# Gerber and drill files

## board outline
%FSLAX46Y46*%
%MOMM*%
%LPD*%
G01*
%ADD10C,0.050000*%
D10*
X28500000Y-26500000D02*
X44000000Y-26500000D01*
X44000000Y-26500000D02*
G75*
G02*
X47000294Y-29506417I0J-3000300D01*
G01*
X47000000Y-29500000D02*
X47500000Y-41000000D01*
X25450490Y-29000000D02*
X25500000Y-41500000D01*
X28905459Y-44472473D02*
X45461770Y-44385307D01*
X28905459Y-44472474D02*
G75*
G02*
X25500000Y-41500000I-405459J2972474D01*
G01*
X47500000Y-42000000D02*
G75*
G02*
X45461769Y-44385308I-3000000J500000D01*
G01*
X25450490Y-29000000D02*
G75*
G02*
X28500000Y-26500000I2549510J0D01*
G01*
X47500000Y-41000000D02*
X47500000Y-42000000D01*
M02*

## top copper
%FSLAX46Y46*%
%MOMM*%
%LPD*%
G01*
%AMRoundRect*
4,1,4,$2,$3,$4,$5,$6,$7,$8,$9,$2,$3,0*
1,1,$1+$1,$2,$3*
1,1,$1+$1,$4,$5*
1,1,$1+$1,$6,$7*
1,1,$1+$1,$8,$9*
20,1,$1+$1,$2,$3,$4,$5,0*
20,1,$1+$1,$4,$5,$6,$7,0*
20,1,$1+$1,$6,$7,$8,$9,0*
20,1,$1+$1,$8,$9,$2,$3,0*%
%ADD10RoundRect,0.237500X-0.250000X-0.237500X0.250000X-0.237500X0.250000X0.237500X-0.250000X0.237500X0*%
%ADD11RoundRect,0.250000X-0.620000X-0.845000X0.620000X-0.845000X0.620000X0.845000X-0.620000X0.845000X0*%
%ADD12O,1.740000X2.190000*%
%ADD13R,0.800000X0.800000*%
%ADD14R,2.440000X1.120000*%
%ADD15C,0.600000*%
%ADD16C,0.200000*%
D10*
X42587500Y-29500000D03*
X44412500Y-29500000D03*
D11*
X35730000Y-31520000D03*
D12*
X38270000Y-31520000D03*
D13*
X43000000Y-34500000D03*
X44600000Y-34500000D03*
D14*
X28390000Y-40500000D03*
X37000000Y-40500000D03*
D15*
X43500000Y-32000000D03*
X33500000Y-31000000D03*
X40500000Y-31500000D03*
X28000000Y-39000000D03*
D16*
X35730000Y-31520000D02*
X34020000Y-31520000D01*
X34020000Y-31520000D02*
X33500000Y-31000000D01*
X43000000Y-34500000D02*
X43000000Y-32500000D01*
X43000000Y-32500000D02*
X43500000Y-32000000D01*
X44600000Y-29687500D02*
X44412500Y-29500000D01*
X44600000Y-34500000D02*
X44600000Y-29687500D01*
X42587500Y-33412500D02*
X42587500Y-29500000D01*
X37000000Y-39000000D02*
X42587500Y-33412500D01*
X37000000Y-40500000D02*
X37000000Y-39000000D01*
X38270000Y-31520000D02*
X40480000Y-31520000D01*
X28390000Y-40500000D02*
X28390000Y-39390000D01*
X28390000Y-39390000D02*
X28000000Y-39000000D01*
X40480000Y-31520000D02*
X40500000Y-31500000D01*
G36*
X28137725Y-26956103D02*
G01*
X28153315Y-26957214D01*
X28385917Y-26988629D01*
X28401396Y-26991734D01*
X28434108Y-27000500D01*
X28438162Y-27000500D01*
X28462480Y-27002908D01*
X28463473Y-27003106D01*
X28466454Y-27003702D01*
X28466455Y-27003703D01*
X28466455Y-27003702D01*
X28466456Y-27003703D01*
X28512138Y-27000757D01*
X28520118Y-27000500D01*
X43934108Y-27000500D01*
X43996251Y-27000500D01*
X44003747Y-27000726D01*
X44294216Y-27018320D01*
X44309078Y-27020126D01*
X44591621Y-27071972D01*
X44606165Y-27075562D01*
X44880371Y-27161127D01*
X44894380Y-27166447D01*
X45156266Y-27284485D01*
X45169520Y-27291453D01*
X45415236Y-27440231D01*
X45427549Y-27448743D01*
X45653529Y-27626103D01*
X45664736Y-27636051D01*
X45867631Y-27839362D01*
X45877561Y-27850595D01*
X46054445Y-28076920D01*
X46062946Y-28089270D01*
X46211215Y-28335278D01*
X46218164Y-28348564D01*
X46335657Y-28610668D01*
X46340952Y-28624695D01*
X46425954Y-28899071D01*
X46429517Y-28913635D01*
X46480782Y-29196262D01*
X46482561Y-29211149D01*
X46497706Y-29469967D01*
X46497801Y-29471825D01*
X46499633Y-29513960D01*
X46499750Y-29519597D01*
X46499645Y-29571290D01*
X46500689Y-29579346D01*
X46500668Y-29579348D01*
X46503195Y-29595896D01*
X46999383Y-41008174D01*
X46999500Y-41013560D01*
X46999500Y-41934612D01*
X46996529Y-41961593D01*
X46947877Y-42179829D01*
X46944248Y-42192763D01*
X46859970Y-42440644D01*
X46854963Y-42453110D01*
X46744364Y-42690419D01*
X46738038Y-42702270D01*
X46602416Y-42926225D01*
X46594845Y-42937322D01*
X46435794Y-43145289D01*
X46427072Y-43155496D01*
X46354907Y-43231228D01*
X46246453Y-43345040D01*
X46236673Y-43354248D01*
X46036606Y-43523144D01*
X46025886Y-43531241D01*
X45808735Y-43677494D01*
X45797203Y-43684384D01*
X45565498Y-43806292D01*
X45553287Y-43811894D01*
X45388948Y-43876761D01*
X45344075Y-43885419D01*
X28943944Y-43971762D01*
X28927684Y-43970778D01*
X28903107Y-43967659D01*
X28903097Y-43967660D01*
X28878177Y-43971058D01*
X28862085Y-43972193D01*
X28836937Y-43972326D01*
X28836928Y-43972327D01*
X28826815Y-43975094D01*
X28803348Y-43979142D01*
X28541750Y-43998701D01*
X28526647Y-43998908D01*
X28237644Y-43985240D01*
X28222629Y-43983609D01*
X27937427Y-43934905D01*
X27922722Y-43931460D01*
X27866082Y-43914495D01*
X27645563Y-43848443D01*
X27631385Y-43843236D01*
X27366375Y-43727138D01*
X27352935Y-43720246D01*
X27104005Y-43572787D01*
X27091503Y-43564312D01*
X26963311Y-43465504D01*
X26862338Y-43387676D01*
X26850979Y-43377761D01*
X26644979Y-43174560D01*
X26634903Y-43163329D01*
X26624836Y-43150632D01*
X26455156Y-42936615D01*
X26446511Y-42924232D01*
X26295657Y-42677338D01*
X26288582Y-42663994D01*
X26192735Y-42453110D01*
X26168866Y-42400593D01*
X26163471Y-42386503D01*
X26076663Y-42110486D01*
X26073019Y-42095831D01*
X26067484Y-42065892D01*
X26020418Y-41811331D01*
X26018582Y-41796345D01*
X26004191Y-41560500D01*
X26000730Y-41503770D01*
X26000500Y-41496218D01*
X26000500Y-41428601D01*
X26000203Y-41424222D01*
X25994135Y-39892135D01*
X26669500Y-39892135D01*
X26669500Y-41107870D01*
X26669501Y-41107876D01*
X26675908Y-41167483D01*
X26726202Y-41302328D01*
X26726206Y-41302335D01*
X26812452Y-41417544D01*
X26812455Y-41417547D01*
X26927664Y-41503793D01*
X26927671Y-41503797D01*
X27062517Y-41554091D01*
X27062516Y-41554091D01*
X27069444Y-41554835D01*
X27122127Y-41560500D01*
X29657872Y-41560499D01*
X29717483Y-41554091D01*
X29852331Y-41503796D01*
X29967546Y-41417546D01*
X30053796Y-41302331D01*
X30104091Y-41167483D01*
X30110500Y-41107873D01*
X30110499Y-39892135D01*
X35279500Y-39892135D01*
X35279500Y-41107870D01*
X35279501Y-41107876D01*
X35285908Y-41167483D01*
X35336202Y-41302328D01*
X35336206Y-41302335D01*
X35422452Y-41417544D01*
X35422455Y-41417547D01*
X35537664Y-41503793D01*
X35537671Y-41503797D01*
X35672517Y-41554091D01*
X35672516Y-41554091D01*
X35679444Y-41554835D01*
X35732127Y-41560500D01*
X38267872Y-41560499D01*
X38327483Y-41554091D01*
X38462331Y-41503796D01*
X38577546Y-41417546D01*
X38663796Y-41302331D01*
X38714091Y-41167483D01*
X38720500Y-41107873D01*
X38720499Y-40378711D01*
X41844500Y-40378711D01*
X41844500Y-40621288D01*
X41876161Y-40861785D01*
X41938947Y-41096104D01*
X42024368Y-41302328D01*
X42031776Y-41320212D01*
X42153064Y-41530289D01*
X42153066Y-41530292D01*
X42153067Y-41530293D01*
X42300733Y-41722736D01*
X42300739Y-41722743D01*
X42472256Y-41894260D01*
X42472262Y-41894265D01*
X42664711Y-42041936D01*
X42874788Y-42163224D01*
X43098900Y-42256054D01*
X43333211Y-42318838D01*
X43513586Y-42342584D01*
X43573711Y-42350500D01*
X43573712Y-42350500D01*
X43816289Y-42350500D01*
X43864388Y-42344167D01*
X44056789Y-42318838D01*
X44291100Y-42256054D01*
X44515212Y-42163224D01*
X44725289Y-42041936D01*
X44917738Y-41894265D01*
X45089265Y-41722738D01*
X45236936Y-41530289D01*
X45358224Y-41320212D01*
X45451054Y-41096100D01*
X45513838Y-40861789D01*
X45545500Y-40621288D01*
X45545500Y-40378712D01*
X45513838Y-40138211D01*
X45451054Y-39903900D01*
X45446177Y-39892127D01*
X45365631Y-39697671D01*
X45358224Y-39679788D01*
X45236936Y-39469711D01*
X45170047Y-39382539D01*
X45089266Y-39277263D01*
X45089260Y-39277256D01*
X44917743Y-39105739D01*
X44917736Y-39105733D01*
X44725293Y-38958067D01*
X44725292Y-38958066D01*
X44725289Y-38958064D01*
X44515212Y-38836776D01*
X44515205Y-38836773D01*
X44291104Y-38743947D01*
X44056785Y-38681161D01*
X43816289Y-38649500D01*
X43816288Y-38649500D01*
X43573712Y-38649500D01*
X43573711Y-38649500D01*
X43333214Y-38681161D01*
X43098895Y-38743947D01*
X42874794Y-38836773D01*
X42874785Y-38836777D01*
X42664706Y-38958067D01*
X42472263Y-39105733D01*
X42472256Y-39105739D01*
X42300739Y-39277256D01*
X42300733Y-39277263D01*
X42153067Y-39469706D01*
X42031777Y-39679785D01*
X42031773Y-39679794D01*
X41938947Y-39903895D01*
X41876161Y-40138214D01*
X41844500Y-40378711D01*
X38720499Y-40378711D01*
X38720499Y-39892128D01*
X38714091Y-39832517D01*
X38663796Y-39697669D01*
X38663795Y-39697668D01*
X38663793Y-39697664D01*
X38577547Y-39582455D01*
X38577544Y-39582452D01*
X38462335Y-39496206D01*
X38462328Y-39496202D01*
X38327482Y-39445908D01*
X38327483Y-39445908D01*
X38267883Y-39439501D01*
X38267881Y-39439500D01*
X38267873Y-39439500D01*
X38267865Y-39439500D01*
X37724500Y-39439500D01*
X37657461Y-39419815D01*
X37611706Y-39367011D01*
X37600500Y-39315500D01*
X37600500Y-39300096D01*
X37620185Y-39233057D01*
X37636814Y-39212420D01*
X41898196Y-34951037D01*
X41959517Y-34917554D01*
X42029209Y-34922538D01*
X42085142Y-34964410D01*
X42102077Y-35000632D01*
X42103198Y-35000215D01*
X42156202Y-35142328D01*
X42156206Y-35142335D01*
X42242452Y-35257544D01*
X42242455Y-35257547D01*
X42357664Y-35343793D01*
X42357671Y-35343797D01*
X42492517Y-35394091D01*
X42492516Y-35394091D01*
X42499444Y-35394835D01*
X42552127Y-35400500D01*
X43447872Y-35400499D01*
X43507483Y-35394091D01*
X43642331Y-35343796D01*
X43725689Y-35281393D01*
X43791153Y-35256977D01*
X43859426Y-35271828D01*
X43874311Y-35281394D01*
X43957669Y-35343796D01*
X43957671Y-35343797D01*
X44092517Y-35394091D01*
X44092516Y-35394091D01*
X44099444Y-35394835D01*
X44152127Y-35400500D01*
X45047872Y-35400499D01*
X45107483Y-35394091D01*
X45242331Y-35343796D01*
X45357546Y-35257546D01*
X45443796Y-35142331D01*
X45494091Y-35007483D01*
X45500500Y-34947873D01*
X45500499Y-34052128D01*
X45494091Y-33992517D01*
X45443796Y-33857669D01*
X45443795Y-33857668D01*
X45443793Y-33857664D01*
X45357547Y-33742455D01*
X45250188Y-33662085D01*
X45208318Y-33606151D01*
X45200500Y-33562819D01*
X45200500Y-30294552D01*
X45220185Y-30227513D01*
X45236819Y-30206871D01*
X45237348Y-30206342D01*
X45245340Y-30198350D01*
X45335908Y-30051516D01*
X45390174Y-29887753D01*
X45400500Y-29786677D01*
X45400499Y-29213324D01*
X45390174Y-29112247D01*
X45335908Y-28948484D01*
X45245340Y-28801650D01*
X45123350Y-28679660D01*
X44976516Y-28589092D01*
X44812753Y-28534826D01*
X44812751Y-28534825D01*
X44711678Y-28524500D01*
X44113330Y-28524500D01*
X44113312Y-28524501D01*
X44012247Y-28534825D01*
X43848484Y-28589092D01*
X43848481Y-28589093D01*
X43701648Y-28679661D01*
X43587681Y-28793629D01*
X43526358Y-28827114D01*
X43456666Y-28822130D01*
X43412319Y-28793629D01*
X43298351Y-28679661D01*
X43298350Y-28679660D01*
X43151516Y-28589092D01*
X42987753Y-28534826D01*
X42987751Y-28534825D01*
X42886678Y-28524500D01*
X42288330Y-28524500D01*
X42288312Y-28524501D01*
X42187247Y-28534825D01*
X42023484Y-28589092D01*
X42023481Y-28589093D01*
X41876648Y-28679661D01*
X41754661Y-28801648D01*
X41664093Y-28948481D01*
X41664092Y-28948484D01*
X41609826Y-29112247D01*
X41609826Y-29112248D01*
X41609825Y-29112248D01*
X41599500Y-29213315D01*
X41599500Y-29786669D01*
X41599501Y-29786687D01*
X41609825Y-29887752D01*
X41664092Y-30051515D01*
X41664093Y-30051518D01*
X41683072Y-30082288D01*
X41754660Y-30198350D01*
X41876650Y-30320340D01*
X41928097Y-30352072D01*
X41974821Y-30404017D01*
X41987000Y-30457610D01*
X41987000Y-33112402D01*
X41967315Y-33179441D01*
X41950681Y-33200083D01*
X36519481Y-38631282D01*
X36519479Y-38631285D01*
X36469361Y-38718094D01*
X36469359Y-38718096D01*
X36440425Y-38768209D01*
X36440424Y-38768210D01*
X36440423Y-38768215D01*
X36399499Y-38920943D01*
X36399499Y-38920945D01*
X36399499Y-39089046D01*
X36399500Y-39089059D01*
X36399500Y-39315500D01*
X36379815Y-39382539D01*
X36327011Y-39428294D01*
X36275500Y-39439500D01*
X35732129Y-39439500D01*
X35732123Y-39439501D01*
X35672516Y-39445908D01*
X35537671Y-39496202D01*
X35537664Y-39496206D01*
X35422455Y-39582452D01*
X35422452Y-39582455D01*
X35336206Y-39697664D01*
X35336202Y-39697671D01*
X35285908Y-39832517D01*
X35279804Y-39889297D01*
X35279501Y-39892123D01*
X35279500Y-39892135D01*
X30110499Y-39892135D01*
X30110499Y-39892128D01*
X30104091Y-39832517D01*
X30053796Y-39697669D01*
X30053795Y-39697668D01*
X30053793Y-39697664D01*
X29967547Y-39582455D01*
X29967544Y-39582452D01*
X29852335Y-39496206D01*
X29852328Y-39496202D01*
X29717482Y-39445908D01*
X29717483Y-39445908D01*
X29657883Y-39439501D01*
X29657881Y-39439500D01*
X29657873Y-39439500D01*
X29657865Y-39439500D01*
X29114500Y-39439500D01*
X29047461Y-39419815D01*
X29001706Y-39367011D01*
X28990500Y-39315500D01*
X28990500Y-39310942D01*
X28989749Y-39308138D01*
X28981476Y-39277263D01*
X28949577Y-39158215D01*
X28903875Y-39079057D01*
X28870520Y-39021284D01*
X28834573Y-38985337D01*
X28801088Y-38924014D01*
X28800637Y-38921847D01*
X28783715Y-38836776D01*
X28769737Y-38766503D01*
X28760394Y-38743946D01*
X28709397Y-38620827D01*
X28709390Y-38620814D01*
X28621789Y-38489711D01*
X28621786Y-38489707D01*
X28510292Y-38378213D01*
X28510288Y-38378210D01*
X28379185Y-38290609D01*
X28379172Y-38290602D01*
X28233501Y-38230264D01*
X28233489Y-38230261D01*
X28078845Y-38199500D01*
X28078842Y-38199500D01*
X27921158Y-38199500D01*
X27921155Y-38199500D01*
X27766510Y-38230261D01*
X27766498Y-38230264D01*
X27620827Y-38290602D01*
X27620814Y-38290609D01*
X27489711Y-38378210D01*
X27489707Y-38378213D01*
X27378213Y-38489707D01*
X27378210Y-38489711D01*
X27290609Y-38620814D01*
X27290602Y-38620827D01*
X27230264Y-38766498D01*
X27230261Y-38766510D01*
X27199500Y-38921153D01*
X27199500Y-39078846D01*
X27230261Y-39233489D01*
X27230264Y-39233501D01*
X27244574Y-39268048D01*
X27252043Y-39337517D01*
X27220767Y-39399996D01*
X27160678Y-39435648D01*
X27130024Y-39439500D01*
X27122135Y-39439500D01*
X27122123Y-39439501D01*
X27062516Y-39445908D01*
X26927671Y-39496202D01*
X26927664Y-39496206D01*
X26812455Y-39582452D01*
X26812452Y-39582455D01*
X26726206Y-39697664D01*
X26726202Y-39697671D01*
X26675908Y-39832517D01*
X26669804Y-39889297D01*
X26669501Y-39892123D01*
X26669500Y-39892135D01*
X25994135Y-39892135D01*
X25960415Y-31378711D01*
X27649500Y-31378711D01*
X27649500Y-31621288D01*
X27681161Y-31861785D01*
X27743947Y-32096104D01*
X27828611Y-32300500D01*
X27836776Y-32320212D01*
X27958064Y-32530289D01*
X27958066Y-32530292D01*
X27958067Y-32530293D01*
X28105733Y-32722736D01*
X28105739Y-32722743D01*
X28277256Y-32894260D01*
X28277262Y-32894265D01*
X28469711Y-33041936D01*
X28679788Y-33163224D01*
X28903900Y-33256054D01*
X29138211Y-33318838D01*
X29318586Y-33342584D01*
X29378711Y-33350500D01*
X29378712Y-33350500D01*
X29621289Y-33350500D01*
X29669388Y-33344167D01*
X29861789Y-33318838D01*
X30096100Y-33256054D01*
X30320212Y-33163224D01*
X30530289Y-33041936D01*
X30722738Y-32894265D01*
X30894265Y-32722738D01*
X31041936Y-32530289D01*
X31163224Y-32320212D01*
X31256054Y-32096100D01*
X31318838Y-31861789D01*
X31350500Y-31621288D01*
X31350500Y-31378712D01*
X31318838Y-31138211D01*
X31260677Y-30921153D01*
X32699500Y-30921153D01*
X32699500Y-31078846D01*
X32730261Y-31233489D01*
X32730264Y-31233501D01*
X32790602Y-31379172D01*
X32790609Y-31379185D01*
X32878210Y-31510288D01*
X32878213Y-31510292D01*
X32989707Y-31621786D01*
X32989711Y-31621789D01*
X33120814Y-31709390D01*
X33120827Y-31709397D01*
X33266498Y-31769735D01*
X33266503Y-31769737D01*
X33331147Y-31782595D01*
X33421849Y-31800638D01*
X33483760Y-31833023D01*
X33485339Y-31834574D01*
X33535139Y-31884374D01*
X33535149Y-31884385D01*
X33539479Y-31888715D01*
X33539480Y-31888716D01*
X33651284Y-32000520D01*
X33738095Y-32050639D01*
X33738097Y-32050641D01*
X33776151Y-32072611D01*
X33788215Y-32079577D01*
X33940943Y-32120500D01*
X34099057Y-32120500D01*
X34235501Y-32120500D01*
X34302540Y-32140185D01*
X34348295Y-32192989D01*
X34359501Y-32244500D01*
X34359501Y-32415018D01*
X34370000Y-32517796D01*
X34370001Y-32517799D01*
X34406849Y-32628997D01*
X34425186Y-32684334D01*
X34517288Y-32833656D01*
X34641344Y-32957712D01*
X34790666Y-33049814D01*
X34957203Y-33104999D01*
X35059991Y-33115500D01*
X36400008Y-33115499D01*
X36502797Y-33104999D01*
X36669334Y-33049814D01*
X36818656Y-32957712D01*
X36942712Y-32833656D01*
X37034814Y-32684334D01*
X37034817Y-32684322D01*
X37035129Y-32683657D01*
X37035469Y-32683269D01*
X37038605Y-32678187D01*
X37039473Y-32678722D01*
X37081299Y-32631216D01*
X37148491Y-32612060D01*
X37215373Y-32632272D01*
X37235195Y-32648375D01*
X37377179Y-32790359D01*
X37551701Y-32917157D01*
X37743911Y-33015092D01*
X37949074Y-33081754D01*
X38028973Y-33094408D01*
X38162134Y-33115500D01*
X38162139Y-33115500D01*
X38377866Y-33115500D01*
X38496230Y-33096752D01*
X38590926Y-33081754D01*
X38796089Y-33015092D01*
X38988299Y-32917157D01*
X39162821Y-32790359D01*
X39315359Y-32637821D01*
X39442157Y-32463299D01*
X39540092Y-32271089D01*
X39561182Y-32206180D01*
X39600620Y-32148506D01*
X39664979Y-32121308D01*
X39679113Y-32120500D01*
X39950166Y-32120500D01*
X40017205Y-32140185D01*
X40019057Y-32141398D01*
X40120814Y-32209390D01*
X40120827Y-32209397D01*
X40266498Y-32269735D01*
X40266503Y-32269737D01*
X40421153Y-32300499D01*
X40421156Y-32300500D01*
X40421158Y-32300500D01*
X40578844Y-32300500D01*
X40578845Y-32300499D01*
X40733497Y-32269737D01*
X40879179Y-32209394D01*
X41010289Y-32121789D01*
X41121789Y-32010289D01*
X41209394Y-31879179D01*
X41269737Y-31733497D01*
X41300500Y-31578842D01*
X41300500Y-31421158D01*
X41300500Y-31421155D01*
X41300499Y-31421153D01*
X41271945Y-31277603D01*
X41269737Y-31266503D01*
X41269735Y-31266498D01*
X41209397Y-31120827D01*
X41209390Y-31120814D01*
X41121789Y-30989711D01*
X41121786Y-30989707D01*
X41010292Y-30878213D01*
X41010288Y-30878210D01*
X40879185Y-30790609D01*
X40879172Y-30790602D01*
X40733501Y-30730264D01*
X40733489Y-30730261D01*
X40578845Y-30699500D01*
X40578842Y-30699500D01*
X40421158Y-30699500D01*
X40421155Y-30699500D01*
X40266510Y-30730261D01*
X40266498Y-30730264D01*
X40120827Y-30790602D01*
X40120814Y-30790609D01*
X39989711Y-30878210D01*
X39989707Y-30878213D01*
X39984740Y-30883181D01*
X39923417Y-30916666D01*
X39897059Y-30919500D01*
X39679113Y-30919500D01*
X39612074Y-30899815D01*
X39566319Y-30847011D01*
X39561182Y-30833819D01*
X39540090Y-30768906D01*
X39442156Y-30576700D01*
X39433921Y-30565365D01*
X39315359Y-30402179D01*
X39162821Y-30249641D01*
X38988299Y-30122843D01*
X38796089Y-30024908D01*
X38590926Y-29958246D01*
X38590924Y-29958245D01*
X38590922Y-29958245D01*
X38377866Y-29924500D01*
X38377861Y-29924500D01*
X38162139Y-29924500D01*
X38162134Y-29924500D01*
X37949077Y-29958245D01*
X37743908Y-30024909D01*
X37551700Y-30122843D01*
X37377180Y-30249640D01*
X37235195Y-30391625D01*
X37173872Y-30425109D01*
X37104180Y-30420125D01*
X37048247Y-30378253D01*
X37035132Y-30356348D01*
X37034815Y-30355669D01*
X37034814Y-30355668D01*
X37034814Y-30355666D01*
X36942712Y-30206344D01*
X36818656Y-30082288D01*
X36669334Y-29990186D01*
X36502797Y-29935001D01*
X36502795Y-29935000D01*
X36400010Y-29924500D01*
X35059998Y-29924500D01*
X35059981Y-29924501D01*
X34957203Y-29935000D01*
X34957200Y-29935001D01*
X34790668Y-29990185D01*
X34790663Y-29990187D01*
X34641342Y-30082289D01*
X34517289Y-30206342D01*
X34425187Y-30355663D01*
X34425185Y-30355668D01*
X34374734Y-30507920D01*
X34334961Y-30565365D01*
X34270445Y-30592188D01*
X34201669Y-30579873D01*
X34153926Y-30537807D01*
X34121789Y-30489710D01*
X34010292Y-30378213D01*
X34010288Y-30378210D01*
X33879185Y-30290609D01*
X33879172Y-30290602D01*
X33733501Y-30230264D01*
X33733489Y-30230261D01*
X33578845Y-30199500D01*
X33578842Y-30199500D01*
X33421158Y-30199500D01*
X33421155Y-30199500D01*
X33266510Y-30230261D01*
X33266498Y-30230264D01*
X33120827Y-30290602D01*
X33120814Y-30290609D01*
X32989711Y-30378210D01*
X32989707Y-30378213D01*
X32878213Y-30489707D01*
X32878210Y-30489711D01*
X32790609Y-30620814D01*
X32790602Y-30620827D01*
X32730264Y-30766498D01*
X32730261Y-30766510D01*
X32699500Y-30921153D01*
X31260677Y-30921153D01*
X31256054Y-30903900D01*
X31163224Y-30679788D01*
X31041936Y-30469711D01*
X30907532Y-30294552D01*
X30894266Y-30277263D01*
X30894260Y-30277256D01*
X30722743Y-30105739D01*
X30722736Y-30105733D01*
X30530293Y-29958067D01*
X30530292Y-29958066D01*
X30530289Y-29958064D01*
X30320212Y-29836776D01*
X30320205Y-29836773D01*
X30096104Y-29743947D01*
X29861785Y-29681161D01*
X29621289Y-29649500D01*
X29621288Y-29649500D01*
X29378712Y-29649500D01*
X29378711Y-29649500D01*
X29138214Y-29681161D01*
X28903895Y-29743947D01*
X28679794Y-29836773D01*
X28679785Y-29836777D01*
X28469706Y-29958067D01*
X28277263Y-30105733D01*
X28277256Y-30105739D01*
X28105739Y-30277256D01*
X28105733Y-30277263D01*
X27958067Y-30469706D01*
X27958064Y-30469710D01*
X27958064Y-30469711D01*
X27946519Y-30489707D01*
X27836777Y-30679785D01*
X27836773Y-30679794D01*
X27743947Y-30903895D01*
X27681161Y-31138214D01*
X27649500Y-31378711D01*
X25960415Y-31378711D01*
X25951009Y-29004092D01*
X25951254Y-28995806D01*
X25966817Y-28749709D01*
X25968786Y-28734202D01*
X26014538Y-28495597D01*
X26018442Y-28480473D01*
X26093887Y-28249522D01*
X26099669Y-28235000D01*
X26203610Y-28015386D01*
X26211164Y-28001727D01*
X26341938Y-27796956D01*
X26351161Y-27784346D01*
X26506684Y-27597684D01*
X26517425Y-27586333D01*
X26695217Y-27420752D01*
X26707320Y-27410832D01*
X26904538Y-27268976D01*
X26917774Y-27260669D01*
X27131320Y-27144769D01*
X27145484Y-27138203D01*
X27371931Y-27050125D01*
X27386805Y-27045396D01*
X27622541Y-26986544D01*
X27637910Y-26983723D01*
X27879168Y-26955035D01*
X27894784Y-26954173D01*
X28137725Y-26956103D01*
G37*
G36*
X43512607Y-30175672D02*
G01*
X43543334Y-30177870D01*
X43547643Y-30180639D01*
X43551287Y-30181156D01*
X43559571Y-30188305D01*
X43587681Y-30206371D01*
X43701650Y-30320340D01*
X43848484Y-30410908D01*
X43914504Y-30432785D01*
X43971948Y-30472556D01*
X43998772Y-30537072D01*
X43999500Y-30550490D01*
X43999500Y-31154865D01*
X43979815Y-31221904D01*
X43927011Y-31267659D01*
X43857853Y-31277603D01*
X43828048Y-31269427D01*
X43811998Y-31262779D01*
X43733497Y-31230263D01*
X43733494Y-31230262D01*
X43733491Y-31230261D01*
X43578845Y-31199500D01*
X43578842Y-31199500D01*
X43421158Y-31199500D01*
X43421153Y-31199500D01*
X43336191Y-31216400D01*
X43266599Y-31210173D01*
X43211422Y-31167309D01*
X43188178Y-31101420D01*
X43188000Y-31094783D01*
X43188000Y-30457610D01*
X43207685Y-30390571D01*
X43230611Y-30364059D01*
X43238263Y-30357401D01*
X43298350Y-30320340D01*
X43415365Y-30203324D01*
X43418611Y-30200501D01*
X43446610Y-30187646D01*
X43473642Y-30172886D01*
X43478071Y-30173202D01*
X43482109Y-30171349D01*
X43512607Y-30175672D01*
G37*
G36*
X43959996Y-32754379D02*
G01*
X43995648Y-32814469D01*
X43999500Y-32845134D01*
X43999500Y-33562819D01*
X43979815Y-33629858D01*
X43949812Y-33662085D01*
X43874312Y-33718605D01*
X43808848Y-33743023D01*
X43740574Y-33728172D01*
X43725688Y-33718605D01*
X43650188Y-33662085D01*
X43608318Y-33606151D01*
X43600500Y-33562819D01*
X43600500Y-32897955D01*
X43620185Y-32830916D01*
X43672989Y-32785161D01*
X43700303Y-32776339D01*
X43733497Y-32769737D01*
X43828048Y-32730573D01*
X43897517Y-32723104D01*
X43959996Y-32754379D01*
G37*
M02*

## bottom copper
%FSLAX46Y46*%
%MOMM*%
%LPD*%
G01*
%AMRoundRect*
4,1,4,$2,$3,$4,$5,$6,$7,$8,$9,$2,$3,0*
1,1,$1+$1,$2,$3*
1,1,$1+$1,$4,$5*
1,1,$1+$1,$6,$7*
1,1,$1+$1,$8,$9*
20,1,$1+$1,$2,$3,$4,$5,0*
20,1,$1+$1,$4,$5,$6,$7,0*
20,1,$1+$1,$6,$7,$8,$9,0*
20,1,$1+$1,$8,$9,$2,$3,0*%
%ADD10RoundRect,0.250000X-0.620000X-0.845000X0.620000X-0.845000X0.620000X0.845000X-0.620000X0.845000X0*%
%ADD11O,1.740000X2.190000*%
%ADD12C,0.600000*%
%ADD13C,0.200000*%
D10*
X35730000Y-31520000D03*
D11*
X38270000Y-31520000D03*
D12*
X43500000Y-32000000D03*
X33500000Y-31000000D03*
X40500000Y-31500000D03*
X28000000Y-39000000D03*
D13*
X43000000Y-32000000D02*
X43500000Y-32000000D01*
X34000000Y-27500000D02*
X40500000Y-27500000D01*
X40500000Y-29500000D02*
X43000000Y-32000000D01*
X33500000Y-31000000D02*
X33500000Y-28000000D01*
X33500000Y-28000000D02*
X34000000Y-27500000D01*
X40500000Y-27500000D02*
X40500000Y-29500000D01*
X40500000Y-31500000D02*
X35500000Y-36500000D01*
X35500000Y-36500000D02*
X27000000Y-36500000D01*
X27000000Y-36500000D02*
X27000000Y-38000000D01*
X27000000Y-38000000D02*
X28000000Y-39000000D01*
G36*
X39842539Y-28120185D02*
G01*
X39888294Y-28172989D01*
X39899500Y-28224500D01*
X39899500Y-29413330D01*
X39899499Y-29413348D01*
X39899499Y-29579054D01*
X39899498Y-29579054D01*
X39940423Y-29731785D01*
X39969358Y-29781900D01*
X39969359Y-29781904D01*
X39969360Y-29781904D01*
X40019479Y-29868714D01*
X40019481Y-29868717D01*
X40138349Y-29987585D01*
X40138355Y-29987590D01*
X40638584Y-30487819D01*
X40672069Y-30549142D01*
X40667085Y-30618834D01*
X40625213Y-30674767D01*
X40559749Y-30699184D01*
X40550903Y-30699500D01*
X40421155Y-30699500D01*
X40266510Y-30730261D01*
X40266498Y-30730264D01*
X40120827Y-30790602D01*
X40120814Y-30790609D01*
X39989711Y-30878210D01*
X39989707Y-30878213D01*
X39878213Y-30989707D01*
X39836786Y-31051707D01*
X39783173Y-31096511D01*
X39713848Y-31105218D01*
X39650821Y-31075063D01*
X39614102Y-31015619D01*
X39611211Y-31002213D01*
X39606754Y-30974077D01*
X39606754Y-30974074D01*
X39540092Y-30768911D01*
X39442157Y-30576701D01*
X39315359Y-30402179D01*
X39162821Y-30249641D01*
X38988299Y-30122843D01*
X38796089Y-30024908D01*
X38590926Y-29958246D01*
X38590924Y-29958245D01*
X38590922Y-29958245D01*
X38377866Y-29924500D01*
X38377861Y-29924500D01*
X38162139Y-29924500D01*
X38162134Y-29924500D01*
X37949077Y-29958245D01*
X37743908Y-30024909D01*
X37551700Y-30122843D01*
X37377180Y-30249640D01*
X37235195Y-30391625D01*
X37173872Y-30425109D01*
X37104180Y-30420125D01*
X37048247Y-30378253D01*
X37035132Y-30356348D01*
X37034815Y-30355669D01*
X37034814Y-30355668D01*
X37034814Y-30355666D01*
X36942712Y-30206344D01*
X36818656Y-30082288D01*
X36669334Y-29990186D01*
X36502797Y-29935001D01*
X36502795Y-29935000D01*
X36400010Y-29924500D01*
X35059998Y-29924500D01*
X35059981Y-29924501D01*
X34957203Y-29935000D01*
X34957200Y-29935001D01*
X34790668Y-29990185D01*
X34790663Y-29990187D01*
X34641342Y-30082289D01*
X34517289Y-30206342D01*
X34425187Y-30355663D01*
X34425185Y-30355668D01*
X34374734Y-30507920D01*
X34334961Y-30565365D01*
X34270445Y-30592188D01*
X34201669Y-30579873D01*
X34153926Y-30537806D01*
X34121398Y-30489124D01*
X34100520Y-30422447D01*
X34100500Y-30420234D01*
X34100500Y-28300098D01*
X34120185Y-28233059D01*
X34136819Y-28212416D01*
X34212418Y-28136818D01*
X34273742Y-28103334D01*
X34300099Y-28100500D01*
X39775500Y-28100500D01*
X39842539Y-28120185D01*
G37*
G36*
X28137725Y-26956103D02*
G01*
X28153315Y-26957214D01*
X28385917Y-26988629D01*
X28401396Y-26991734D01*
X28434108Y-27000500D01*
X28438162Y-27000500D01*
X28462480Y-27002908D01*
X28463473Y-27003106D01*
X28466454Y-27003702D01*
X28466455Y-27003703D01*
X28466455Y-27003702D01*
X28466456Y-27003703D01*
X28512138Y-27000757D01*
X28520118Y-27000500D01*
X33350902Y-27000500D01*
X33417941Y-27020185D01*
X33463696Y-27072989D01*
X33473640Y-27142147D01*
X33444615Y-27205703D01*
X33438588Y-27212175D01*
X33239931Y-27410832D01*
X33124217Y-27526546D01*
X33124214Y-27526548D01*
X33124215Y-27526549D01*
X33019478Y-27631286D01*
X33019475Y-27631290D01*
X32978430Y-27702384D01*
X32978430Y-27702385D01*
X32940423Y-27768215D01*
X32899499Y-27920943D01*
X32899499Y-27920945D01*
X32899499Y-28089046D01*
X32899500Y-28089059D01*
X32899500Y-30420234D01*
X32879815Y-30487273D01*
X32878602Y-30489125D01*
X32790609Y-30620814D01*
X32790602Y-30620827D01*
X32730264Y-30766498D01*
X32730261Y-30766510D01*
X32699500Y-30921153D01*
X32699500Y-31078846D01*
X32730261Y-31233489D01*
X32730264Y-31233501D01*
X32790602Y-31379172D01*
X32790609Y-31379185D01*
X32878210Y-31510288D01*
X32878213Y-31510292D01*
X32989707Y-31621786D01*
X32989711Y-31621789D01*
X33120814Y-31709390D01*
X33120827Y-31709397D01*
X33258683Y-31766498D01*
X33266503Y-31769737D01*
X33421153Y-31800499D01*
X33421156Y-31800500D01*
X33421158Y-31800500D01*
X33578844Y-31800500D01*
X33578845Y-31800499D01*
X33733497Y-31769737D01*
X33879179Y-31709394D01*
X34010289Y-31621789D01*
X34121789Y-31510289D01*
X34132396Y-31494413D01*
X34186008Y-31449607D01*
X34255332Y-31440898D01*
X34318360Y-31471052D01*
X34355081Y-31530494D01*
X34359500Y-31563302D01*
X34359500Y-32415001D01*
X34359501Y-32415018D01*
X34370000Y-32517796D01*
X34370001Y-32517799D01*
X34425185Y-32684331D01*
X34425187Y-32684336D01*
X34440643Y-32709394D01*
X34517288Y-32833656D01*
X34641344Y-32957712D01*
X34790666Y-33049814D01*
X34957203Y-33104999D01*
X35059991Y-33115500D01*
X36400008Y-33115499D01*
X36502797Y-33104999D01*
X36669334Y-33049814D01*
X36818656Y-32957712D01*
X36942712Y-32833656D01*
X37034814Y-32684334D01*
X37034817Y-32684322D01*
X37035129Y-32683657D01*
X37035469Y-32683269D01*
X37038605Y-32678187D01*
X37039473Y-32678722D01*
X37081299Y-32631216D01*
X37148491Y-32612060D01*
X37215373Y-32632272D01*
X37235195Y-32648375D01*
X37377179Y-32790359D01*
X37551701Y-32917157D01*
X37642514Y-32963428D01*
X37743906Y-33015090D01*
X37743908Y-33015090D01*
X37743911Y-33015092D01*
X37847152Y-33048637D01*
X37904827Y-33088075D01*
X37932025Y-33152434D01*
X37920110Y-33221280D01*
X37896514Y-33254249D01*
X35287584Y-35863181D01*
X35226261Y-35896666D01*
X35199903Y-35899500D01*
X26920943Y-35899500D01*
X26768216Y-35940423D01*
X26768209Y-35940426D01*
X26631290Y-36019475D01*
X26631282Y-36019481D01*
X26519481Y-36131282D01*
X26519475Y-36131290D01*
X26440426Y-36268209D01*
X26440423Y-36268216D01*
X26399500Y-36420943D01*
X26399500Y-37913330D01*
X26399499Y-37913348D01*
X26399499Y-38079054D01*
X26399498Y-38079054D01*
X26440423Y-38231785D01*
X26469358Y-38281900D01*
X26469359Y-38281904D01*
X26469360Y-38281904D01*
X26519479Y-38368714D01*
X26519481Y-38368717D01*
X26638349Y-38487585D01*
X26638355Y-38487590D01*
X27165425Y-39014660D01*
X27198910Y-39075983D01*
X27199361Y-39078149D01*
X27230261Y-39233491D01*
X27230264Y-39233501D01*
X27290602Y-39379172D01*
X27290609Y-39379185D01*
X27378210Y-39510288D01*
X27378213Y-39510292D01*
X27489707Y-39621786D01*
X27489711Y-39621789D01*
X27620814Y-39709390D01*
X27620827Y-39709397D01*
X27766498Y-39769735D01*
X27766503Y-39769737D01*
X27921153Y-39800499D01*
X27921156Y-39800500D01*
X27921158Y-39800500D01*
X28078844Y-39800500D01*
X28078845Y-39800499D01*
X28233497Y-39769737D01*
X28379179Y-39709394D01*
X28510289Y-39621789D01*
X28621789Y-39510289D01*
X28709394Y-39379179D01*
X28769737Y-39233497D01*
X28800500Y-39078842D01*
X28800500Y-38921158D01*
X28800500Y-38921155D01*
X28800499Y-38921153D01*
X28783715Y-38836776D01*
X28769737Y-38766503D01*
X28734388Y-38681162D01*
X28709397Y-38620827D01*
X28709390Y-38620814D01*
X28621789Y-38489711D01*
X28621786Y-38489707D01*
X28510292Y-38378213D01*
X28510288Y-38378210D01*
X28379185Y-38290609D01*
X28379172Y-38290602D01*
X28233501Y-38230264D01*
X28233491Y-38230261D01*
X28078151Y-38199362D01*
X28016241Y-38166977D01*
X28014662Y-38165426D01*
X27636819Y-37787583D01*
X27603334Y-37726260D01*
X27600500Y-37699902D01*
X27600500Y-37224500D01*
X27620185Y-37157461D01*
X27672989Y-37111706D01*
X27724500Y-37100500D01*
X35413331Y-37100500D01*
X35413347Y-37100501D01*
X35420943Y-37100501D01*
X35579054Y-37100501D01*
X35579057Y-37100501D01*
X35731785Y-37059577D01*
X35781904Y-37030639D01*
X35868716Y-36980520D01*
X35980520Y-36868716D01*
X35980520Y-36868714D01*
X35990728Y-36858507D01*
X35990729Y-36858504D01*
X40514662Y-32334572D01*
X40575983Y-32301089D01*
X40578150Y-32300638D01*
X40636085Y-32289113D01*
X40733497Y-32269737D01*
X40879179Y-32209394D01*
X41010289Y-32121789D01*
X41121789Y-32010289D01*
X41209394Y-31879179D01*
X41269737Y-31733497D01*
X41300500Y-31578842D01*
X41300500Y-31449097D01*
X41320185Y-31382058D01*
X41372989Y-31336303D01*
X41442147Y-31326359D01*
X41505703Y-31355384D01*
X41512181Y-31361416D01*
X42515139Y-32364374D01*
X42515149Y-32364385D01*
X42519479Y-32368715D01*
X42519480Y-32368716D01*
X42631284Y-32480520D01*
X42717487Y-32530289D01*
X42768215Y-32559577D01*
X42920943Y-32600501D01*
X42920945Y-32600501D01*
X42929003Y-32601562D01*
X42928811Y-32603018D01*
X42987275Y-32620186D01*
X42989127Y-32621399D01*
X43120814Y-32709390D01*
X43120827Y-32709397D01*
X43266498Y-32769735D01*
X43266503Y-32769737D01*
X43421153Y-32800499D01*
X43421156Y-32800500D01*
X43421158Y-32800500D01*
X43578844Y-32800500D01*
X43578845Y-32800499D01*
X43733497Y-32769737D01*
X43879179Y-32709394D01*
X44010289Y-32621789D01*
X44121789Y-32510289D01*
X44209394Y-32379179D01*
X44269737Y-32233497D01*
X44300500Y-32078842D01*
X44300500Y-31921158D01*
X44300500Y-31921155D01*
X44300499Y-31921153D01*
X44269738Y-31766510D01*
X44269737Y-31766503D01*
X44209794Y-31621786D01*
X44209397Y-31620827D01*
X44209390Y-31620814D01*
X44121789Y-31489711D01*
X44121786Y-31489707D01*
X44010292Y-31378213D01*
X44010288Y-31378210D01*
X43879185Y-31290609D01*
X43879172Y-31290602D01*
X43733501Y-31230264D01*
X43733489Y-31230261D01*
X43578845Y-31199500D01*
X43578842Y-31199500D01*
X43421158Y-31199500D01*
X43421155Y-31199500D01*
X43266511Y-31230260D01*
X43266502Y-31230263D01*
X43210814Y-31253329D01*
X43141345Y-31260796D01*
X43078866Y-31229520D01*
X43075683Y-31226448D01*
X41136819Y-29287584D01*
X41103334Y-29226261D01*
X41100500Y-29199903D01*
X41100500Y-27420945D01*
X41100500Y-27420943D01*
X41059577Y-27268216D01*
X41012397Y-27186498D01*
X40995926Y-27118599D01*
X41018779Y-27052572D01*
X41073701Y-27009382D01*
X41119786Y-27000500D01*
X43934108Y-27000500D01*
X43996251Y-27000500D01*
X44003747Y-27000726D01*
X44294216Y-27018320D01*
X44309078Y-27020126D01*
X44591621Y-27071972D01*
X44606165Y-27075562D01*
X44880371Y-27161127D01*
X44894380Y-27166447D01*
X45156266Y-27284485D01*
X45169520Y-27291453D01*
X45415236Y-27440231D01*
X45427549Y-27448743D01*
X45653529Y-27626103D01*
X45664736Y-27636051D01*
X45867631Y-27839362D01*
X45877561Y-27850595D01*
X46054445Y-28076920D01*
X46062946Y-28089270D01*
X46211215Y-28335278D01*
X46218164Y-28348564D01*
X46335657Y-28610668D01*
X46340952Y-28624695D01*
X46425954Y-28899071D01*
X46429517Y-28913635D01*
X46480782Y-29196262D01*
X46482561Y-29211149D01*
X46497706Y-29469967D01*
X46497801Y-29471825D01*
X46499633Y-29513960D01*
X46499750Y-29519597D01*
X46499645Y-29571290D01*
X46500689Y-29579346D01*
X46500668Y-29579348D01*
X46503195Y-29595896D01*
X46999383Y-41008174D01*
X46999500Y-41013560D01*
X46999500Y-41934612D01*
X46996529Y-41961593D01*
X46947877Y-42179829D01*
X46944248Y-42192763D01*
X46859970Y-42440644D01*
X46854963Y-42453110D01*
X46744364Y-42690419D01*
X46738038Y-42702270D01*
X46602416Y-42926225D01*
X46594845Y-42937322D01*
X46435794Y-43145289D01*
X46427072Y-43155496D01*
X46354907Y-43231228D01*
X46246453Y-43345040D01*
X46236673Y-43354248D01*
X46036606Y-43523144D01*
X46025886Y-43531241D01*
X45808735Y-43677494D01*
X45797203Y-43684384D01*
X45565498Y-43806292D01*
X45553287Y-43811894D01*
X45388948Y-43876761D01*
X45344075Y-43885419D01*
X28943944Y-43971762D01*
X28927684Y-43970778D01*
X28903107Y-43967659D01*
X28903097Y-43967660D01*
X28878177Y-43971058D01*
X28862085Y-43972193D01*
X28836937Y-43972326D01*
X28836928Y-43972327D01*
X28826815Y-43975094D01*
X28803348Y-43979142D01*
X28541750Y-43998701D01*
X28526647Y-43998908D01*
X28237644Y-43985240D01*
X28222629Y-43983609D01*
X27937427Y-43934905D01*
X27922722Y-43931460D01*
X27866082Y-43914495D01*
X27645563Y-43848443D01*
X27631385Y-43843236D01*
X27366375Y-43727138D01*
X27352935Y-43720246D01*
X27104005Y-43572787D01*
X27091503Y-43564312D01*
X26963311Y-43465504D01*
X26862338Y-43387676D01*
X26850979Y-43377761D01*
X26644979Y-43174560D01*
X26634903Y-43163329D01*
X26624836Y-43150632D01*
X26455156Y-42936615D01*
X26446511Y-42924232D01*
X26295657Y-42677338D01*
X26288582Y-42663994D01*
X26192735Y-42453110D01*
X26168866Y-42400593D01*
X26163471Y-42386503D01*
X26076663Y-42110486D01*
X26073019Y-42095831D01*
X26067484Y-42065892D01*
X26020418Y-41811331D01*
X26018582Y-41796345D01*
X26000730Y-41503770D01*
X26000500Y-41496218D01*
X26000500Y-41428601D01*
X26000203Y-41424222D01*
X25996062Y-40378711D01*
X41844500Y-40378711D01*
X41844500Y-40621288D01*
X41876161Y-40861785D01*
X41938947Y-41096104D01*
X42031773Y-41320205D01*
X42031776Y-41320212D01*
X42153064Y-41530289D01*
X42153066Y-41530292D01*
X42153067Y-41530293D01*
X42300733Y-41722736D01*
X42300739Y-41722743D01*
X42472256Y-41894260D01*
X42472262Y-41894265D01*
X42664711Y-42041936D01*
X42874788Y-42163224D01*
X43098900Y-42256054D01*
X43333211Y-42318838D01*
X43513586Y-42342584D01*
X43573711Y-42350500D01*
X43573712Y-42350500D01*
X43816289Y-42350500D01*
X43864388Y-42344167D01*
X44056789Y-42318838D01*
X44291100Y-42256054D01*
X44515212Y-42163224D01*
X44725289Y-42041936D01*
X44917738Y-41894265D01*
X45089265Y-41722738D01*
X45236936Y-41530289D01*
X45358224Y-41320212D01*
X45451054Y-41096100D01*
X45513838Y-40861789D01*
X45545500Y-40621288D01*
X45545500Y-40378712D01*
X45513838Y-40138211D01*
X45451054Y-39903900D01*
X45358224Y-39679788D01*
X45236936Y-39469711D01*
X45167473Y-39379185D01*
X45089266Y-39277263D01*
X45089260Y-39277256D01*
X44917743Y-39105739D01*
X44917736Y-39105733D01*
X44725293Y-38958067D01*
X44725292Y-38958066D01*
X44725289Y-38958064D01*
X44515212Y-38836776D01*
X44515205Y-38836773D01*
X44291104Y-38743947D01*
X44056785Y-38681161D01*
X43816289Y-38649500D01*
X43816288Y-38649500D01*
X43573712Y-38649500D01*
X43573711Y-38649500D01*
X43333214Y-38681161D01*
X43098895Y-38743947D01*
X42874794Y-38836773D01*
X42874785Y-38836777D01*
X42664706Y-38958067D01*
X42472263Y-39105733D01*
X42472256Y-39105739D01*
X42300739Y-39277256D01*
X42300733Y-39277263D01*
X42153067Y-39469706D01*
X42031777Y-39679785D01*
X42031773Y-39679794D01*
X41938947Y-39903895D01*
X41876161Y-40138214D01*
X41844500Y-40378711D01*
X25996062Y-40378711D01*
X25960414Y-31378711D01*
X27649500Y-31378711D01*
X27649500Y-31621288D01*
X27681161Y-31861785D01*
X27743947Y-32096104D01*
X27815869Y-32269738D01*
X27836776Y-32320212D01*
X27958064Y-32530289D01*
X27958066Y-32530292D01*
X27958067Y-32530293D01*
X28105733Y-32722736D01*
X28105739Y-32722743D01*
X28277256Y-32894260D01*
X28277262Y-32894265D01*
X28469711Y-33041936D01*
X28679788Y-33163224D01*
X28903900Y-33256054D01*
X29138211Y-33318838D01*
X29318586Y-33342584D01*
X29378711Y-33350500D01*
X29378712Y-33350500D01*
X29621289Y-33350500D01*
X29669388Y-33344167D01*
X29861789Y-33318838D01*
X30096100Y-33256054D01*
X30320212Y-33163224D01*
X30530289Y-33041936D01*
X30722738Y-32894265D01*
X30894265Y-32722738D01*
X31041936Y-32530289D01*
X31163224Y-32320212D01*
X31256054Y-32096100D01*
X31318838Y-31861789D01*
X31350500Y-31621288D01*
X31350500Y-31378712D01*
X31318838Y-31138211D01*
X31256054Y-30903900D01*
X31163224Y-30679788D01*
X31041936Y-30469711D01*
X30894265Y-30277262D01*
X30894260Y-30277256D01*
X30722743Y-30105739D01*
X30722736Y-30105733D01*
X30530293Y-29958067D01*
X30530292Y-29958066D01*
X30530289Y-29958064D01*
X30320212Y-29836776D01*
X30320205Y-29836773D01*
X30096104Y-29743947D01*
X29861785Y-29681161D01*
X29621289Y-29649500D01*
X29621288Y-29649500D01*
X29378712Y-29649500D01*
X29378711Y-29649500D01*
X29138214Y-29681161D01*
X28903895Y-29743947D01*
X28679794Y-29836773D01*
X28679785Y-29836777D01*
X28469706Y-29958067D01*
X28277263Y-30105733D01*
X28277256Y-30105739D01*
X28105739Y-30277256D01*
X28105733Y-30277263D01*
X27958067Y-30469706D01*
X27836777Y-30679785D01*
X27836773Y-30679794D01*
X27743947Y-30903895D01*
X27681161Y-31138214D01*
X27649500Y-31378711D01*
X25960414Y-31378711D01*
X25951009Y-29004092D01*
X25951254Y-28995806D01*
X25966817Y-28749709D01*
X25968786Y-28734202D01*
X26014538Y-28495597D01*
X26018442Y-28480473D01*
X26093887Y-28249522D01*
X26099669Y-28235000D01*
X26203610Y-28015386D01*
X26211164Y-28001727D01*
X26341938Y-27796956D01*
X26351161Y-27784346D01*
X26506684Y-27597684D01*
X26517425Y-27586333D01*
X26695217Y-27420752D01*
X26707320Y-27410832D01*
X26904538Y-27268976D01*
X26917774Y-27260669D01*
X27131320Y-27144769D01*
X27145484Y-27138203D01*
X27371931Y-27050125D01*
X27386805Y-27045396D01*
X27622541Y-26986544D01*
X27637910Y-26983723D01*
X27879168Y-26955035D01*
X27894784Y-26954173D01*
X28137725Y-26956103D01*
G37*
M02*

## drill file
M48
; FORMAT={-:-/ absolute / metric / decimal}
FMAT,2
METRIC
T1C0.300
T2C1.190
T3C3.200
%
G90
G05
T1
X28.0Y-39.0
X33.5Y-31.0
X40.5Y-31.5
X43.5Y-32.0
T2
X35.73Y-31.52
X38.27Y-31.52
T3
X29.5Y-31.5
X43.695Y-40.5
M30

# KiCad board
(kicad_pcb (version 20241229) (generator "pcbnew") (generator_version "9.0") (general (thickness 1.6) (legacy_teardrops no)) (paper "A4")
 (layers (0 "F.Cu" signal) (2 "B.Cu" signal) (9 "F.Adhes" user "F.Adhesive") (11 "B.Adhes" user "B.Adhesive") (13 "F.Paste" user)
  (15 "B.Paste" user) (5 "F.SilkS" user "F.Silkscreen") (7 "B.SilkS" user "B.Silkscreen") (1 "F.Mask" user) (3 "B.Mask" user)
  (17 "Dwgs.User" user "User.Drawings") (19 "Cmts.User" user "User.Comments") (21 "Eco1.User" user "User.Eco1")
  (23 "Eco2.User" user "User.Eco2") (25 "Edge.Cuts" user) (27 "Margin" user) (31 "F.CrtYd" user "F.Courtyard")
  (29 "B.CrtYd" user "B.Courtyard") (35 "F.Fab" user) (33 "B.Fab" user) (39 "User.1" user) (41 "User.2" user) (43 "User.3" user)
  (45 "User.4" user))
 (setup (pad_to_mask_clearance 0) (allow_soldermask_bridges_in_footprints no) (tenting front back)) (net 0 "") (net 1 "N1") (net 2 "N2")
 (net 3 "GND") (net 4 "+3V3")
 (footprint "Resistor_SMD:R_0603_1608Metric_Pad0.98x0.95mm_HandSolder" (layer "F.Cu") (at 43.5 29.5)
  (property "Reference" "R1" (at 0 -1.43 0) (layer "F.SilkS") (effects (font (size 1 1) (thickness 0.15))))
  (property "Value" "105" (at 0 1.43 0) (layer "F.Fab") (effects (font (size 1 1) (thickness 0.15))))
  (pad "1" smd roundrect (at -0.9125 0) (size 0.975 0.95) (layers "F.Cu" "F.Mask" "F.Paste") (roundrect_rratio 0.25) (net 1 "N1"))
  (pad "2" smd roundrect (at 0.9125 0) (size 0.975 0.95) (layers "F.Cu" "F.Mask" "F.Paste") (roundrect_rratio 0.25) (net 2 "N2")))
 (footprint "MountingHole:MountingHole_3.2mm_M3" (layer "F.Cu") (at 43.695 40.5)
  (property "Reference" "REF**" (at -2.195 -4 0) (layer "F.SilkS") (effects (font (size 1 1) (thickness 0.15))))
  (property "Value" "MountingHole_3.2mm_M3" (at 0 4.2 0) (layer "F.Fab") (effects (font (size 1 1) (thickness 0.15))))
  (pad "" np_thru_hole circle (at 0 0) (size 3.2 3.2) (drill 3.2) (layers "*.Cu" "*.Mask")))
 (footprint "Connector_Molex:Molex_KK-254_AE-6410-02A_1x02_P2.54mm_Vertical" (layer "F.Cu") (at 35.73 31.52)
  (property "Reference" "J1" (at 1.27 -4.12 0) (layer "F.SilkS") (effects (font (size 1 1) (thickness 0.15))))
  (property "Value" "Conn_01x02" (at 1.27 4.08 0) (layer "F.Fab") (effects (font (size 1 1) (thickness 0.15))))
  (pad "1" thru_hole roundrect (at 0 0) (size 1.74 2.19) (drill 1.19) (layers "*.Cu" "*.Mask") (remove_unused_layers no)
   (roundrect_rratio 0.143678) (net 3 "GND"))
  (pad "2" thru_hole oval (at 2.54 0) (size 1.74 2.19) (drill 1.19) (layers "*.Cu" "*.Mask") (remove_unused_layers no) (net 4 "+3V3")))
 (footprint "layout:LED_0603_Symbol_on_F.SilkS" (layer "F.Cu") (at 43.8 34.5)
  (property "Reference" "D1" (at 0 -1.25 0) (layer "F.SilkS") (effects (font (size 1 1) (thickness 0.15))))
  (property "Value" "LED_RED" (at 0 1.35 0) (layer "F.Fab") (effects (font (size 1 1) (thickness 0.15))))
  (pad "1" smd rect (at -0.8 0 180) (size 0.8 0.8) (layers "F.Cu" "F.Mask" "F.Paste") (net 3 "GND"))
  (pad "2" smd rect (at 0.8 0 180) (size 0.8 0.8) (layers "F.Cu" "F.Mask" "F.Paste") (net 2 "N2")))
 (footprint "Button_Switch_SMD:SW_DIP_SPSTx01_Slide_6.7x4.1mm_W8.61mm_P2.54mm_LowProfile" (layer "F.Cu") (at 32.695 40.5)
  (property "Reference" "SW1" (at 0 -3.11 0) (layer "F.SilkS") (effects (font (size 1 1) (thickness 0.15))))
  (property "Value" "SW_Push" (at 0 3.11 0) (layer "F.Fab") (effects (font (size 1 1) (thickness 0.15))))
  (pad "1" smd rect (at -4.305 0) (size 2.44 1.12) (layers "F.Cu" "F.Mask" "F.Paste") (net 4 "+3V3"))
  (pad "2" smd rect (at 4.305 0) (size 2.44 1.12) (layers "F.Cu" "F.Mask" "F.Paste") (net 1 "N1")))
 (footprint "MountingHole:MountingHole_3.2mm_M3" (layer "F.Cu") (at 29.5 31.5)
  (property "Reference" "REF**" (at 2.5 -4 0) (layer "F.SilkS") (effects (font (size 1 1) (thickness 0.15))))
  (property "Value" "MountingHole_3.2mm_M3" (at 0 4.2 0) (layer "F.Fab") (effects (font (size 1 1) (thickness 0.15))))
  (pad "" np_thru_hole circle (at 0 0) (size 3.2 3.2) (drill 3.2) (layers "*.Cu" "*.Mask")))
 (gr_line (start 28.5 26.5) (end 44 26.5) (stroke (width 0.05) (type default)) (layer "Edge.Cuts"))
 (gr_arc (start 44 26.5) (mid 46.123689 27.380932) (end 47.000279 29.506417) (stroke (width 0.05) (type default)) (layer "Edge.Cuts"))
 (gr_line (start 47 29.5) (end 47.5 41) (stroke (width 0.05) (type default)) (layer "Edge.Cuts"))
 (gr_line (start 25.45049 29) (end 25.5 41.5) (stroke (width 0.05) (type default)) (layer "Edge.Cuts"))
 (gr_line (start 28.905459 44.472473) (end 45.46177 44.385307) (stroke (width 0.05) (type default)) (layer "Edge.Cuts"))
 (gr_arc (start 28.905459 44.472474) (mid 26.527233 43.76013) (end 25.5 41.5) (stroke (width 0.05) (type default)) (layer "Edge.Cuts"))
 (gr_arc (start 47.5 42) (mid 46.812213 43.475772) (end 45.461769 44.385307) (stroke (width 0.05) (type default)) (layer "Edge.Cuts"))
 (gr_arc (start 25.45049 29) (mid 26.383639 27.028356) (end 28.5 26.5) (stroke (width 0.05) (type default)) (layer "Edge.Cuts"))
 (gr_line (start 47.5 41) (end 47.5 42) (stroke (width 0.05) (type default)) (layer "Edge.Cuts"))
 (segment (start 35.73 31.52) (end 34.02 31.52) (width 0.2) (layer "F.Cu") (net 3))
 (segment (start 34.02 31.52) (end 33.5 31) (width 0.2) (layer "F.Cu") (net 3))
 (segment (start 43 34.5) (end 43 32.5) (width 0.2) (layer "F.Cu") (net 3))
 (segment (start 43 32.5) (end 43.5 32) (width 0.2) (layer "F.Cu") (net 3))
 (via (at 43.5 32) (size 0.6) (drill 0.3) (layers "F.Cu" "B.Cu") (free yes) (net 3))
 (via (at 33.5 31) (size 0.6) (drill 0.3) (layers "F.Cu" "B.Cu") (free yes) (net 3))
 (segment (start 43 32) (end 43.5 32) (width 0.2) (layer "B.Cu") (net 3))
 (segment (start 34 27.5) (end 40.5 27.5) (width 0.2) (layer "B.Cu") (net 3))
 (segment (start 40.5 29.5) (end 43 32) (width 0.2) (layer "B.Cu") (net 3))
 (segment (start 33.5 31) (end 33.5 28) (width 0.2) (layer "B.Cu") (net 3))
 (segment (start 33.5 28) (end 34 27.5) (width 0.2) (layer "B.Cu") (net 3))
 (segment (start 40.5 27.5) (end 40.5 29.5) (width 0.2) (layer "B.Cu") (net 3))
 (segment (start 44.6 29.6875) (end 44.4125 29.5) (width 0.2) (layer "F.Cu") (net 2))
 (segment (start 44.6 34.5) (end 44.6 29.6875) (width 0.2) (layer "F.Cu") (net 2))
 (segment (start 42.5875 33.4125) (end 42.5875 29.5) (width 0.2) (layer "F.Cu") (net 1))
 (segment (start 37 39) (end 42.5875 33.4125) (width 0.2) (layer "F.Cu") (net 1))
 (segment (start 37 40.5) (end 37 39) (width 0.2) (layer "F.Cu") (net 1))
 (segment (start 38.27 31.52) (end 40.48 31.52) (width 0.2) (layer "F.Cu") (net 4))
 (segment (start 28.39 40.5) (end 28.39 39.39) (width 0.2) (layer "F.Cu") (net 4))
 (segment (start 28.39 39.39) (end 28 39) (width 0.2) (layer "F.Cu") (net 4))
 (segment (start 40.48 31.52) (end 40.5 31.5) (width 0.2) (layer "F.Cu") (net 4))
 (via (at 40.5 31.5) (size 0.6) (drill 0.3) (layers "F.Cu" "B.Cu") (free yes) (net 4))
 (via (at 28 39) (size 0.6) (drill 0.3) (layers "F.Cu" "B.Cu") (free yes) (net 4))
 (segment (start 40.5 31.5) (end 35.5 36.5) (width 0.2) (layer "B.Cu") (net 4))
 (segment (start 35.5 36.5) (end 27 36.5) (width 0.2) (layer "B.Cu") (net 4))
 (segment (start 27 36.5) (end 27 38) (width 0.2) (layer "B.Cu") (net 4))
 (segment (start 27 38) (end 28 39) (width 0.2) (layer "B.Cu") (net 4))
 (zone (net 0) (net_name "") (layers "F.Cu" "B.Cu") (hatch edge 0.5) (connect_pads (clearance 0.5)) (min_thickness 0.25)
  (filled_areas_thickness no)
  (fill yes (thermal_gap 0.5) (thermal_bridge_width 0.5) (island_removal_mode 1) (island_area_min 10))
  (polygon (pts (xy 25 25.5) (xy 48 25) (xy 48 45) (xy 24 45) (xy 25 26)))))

